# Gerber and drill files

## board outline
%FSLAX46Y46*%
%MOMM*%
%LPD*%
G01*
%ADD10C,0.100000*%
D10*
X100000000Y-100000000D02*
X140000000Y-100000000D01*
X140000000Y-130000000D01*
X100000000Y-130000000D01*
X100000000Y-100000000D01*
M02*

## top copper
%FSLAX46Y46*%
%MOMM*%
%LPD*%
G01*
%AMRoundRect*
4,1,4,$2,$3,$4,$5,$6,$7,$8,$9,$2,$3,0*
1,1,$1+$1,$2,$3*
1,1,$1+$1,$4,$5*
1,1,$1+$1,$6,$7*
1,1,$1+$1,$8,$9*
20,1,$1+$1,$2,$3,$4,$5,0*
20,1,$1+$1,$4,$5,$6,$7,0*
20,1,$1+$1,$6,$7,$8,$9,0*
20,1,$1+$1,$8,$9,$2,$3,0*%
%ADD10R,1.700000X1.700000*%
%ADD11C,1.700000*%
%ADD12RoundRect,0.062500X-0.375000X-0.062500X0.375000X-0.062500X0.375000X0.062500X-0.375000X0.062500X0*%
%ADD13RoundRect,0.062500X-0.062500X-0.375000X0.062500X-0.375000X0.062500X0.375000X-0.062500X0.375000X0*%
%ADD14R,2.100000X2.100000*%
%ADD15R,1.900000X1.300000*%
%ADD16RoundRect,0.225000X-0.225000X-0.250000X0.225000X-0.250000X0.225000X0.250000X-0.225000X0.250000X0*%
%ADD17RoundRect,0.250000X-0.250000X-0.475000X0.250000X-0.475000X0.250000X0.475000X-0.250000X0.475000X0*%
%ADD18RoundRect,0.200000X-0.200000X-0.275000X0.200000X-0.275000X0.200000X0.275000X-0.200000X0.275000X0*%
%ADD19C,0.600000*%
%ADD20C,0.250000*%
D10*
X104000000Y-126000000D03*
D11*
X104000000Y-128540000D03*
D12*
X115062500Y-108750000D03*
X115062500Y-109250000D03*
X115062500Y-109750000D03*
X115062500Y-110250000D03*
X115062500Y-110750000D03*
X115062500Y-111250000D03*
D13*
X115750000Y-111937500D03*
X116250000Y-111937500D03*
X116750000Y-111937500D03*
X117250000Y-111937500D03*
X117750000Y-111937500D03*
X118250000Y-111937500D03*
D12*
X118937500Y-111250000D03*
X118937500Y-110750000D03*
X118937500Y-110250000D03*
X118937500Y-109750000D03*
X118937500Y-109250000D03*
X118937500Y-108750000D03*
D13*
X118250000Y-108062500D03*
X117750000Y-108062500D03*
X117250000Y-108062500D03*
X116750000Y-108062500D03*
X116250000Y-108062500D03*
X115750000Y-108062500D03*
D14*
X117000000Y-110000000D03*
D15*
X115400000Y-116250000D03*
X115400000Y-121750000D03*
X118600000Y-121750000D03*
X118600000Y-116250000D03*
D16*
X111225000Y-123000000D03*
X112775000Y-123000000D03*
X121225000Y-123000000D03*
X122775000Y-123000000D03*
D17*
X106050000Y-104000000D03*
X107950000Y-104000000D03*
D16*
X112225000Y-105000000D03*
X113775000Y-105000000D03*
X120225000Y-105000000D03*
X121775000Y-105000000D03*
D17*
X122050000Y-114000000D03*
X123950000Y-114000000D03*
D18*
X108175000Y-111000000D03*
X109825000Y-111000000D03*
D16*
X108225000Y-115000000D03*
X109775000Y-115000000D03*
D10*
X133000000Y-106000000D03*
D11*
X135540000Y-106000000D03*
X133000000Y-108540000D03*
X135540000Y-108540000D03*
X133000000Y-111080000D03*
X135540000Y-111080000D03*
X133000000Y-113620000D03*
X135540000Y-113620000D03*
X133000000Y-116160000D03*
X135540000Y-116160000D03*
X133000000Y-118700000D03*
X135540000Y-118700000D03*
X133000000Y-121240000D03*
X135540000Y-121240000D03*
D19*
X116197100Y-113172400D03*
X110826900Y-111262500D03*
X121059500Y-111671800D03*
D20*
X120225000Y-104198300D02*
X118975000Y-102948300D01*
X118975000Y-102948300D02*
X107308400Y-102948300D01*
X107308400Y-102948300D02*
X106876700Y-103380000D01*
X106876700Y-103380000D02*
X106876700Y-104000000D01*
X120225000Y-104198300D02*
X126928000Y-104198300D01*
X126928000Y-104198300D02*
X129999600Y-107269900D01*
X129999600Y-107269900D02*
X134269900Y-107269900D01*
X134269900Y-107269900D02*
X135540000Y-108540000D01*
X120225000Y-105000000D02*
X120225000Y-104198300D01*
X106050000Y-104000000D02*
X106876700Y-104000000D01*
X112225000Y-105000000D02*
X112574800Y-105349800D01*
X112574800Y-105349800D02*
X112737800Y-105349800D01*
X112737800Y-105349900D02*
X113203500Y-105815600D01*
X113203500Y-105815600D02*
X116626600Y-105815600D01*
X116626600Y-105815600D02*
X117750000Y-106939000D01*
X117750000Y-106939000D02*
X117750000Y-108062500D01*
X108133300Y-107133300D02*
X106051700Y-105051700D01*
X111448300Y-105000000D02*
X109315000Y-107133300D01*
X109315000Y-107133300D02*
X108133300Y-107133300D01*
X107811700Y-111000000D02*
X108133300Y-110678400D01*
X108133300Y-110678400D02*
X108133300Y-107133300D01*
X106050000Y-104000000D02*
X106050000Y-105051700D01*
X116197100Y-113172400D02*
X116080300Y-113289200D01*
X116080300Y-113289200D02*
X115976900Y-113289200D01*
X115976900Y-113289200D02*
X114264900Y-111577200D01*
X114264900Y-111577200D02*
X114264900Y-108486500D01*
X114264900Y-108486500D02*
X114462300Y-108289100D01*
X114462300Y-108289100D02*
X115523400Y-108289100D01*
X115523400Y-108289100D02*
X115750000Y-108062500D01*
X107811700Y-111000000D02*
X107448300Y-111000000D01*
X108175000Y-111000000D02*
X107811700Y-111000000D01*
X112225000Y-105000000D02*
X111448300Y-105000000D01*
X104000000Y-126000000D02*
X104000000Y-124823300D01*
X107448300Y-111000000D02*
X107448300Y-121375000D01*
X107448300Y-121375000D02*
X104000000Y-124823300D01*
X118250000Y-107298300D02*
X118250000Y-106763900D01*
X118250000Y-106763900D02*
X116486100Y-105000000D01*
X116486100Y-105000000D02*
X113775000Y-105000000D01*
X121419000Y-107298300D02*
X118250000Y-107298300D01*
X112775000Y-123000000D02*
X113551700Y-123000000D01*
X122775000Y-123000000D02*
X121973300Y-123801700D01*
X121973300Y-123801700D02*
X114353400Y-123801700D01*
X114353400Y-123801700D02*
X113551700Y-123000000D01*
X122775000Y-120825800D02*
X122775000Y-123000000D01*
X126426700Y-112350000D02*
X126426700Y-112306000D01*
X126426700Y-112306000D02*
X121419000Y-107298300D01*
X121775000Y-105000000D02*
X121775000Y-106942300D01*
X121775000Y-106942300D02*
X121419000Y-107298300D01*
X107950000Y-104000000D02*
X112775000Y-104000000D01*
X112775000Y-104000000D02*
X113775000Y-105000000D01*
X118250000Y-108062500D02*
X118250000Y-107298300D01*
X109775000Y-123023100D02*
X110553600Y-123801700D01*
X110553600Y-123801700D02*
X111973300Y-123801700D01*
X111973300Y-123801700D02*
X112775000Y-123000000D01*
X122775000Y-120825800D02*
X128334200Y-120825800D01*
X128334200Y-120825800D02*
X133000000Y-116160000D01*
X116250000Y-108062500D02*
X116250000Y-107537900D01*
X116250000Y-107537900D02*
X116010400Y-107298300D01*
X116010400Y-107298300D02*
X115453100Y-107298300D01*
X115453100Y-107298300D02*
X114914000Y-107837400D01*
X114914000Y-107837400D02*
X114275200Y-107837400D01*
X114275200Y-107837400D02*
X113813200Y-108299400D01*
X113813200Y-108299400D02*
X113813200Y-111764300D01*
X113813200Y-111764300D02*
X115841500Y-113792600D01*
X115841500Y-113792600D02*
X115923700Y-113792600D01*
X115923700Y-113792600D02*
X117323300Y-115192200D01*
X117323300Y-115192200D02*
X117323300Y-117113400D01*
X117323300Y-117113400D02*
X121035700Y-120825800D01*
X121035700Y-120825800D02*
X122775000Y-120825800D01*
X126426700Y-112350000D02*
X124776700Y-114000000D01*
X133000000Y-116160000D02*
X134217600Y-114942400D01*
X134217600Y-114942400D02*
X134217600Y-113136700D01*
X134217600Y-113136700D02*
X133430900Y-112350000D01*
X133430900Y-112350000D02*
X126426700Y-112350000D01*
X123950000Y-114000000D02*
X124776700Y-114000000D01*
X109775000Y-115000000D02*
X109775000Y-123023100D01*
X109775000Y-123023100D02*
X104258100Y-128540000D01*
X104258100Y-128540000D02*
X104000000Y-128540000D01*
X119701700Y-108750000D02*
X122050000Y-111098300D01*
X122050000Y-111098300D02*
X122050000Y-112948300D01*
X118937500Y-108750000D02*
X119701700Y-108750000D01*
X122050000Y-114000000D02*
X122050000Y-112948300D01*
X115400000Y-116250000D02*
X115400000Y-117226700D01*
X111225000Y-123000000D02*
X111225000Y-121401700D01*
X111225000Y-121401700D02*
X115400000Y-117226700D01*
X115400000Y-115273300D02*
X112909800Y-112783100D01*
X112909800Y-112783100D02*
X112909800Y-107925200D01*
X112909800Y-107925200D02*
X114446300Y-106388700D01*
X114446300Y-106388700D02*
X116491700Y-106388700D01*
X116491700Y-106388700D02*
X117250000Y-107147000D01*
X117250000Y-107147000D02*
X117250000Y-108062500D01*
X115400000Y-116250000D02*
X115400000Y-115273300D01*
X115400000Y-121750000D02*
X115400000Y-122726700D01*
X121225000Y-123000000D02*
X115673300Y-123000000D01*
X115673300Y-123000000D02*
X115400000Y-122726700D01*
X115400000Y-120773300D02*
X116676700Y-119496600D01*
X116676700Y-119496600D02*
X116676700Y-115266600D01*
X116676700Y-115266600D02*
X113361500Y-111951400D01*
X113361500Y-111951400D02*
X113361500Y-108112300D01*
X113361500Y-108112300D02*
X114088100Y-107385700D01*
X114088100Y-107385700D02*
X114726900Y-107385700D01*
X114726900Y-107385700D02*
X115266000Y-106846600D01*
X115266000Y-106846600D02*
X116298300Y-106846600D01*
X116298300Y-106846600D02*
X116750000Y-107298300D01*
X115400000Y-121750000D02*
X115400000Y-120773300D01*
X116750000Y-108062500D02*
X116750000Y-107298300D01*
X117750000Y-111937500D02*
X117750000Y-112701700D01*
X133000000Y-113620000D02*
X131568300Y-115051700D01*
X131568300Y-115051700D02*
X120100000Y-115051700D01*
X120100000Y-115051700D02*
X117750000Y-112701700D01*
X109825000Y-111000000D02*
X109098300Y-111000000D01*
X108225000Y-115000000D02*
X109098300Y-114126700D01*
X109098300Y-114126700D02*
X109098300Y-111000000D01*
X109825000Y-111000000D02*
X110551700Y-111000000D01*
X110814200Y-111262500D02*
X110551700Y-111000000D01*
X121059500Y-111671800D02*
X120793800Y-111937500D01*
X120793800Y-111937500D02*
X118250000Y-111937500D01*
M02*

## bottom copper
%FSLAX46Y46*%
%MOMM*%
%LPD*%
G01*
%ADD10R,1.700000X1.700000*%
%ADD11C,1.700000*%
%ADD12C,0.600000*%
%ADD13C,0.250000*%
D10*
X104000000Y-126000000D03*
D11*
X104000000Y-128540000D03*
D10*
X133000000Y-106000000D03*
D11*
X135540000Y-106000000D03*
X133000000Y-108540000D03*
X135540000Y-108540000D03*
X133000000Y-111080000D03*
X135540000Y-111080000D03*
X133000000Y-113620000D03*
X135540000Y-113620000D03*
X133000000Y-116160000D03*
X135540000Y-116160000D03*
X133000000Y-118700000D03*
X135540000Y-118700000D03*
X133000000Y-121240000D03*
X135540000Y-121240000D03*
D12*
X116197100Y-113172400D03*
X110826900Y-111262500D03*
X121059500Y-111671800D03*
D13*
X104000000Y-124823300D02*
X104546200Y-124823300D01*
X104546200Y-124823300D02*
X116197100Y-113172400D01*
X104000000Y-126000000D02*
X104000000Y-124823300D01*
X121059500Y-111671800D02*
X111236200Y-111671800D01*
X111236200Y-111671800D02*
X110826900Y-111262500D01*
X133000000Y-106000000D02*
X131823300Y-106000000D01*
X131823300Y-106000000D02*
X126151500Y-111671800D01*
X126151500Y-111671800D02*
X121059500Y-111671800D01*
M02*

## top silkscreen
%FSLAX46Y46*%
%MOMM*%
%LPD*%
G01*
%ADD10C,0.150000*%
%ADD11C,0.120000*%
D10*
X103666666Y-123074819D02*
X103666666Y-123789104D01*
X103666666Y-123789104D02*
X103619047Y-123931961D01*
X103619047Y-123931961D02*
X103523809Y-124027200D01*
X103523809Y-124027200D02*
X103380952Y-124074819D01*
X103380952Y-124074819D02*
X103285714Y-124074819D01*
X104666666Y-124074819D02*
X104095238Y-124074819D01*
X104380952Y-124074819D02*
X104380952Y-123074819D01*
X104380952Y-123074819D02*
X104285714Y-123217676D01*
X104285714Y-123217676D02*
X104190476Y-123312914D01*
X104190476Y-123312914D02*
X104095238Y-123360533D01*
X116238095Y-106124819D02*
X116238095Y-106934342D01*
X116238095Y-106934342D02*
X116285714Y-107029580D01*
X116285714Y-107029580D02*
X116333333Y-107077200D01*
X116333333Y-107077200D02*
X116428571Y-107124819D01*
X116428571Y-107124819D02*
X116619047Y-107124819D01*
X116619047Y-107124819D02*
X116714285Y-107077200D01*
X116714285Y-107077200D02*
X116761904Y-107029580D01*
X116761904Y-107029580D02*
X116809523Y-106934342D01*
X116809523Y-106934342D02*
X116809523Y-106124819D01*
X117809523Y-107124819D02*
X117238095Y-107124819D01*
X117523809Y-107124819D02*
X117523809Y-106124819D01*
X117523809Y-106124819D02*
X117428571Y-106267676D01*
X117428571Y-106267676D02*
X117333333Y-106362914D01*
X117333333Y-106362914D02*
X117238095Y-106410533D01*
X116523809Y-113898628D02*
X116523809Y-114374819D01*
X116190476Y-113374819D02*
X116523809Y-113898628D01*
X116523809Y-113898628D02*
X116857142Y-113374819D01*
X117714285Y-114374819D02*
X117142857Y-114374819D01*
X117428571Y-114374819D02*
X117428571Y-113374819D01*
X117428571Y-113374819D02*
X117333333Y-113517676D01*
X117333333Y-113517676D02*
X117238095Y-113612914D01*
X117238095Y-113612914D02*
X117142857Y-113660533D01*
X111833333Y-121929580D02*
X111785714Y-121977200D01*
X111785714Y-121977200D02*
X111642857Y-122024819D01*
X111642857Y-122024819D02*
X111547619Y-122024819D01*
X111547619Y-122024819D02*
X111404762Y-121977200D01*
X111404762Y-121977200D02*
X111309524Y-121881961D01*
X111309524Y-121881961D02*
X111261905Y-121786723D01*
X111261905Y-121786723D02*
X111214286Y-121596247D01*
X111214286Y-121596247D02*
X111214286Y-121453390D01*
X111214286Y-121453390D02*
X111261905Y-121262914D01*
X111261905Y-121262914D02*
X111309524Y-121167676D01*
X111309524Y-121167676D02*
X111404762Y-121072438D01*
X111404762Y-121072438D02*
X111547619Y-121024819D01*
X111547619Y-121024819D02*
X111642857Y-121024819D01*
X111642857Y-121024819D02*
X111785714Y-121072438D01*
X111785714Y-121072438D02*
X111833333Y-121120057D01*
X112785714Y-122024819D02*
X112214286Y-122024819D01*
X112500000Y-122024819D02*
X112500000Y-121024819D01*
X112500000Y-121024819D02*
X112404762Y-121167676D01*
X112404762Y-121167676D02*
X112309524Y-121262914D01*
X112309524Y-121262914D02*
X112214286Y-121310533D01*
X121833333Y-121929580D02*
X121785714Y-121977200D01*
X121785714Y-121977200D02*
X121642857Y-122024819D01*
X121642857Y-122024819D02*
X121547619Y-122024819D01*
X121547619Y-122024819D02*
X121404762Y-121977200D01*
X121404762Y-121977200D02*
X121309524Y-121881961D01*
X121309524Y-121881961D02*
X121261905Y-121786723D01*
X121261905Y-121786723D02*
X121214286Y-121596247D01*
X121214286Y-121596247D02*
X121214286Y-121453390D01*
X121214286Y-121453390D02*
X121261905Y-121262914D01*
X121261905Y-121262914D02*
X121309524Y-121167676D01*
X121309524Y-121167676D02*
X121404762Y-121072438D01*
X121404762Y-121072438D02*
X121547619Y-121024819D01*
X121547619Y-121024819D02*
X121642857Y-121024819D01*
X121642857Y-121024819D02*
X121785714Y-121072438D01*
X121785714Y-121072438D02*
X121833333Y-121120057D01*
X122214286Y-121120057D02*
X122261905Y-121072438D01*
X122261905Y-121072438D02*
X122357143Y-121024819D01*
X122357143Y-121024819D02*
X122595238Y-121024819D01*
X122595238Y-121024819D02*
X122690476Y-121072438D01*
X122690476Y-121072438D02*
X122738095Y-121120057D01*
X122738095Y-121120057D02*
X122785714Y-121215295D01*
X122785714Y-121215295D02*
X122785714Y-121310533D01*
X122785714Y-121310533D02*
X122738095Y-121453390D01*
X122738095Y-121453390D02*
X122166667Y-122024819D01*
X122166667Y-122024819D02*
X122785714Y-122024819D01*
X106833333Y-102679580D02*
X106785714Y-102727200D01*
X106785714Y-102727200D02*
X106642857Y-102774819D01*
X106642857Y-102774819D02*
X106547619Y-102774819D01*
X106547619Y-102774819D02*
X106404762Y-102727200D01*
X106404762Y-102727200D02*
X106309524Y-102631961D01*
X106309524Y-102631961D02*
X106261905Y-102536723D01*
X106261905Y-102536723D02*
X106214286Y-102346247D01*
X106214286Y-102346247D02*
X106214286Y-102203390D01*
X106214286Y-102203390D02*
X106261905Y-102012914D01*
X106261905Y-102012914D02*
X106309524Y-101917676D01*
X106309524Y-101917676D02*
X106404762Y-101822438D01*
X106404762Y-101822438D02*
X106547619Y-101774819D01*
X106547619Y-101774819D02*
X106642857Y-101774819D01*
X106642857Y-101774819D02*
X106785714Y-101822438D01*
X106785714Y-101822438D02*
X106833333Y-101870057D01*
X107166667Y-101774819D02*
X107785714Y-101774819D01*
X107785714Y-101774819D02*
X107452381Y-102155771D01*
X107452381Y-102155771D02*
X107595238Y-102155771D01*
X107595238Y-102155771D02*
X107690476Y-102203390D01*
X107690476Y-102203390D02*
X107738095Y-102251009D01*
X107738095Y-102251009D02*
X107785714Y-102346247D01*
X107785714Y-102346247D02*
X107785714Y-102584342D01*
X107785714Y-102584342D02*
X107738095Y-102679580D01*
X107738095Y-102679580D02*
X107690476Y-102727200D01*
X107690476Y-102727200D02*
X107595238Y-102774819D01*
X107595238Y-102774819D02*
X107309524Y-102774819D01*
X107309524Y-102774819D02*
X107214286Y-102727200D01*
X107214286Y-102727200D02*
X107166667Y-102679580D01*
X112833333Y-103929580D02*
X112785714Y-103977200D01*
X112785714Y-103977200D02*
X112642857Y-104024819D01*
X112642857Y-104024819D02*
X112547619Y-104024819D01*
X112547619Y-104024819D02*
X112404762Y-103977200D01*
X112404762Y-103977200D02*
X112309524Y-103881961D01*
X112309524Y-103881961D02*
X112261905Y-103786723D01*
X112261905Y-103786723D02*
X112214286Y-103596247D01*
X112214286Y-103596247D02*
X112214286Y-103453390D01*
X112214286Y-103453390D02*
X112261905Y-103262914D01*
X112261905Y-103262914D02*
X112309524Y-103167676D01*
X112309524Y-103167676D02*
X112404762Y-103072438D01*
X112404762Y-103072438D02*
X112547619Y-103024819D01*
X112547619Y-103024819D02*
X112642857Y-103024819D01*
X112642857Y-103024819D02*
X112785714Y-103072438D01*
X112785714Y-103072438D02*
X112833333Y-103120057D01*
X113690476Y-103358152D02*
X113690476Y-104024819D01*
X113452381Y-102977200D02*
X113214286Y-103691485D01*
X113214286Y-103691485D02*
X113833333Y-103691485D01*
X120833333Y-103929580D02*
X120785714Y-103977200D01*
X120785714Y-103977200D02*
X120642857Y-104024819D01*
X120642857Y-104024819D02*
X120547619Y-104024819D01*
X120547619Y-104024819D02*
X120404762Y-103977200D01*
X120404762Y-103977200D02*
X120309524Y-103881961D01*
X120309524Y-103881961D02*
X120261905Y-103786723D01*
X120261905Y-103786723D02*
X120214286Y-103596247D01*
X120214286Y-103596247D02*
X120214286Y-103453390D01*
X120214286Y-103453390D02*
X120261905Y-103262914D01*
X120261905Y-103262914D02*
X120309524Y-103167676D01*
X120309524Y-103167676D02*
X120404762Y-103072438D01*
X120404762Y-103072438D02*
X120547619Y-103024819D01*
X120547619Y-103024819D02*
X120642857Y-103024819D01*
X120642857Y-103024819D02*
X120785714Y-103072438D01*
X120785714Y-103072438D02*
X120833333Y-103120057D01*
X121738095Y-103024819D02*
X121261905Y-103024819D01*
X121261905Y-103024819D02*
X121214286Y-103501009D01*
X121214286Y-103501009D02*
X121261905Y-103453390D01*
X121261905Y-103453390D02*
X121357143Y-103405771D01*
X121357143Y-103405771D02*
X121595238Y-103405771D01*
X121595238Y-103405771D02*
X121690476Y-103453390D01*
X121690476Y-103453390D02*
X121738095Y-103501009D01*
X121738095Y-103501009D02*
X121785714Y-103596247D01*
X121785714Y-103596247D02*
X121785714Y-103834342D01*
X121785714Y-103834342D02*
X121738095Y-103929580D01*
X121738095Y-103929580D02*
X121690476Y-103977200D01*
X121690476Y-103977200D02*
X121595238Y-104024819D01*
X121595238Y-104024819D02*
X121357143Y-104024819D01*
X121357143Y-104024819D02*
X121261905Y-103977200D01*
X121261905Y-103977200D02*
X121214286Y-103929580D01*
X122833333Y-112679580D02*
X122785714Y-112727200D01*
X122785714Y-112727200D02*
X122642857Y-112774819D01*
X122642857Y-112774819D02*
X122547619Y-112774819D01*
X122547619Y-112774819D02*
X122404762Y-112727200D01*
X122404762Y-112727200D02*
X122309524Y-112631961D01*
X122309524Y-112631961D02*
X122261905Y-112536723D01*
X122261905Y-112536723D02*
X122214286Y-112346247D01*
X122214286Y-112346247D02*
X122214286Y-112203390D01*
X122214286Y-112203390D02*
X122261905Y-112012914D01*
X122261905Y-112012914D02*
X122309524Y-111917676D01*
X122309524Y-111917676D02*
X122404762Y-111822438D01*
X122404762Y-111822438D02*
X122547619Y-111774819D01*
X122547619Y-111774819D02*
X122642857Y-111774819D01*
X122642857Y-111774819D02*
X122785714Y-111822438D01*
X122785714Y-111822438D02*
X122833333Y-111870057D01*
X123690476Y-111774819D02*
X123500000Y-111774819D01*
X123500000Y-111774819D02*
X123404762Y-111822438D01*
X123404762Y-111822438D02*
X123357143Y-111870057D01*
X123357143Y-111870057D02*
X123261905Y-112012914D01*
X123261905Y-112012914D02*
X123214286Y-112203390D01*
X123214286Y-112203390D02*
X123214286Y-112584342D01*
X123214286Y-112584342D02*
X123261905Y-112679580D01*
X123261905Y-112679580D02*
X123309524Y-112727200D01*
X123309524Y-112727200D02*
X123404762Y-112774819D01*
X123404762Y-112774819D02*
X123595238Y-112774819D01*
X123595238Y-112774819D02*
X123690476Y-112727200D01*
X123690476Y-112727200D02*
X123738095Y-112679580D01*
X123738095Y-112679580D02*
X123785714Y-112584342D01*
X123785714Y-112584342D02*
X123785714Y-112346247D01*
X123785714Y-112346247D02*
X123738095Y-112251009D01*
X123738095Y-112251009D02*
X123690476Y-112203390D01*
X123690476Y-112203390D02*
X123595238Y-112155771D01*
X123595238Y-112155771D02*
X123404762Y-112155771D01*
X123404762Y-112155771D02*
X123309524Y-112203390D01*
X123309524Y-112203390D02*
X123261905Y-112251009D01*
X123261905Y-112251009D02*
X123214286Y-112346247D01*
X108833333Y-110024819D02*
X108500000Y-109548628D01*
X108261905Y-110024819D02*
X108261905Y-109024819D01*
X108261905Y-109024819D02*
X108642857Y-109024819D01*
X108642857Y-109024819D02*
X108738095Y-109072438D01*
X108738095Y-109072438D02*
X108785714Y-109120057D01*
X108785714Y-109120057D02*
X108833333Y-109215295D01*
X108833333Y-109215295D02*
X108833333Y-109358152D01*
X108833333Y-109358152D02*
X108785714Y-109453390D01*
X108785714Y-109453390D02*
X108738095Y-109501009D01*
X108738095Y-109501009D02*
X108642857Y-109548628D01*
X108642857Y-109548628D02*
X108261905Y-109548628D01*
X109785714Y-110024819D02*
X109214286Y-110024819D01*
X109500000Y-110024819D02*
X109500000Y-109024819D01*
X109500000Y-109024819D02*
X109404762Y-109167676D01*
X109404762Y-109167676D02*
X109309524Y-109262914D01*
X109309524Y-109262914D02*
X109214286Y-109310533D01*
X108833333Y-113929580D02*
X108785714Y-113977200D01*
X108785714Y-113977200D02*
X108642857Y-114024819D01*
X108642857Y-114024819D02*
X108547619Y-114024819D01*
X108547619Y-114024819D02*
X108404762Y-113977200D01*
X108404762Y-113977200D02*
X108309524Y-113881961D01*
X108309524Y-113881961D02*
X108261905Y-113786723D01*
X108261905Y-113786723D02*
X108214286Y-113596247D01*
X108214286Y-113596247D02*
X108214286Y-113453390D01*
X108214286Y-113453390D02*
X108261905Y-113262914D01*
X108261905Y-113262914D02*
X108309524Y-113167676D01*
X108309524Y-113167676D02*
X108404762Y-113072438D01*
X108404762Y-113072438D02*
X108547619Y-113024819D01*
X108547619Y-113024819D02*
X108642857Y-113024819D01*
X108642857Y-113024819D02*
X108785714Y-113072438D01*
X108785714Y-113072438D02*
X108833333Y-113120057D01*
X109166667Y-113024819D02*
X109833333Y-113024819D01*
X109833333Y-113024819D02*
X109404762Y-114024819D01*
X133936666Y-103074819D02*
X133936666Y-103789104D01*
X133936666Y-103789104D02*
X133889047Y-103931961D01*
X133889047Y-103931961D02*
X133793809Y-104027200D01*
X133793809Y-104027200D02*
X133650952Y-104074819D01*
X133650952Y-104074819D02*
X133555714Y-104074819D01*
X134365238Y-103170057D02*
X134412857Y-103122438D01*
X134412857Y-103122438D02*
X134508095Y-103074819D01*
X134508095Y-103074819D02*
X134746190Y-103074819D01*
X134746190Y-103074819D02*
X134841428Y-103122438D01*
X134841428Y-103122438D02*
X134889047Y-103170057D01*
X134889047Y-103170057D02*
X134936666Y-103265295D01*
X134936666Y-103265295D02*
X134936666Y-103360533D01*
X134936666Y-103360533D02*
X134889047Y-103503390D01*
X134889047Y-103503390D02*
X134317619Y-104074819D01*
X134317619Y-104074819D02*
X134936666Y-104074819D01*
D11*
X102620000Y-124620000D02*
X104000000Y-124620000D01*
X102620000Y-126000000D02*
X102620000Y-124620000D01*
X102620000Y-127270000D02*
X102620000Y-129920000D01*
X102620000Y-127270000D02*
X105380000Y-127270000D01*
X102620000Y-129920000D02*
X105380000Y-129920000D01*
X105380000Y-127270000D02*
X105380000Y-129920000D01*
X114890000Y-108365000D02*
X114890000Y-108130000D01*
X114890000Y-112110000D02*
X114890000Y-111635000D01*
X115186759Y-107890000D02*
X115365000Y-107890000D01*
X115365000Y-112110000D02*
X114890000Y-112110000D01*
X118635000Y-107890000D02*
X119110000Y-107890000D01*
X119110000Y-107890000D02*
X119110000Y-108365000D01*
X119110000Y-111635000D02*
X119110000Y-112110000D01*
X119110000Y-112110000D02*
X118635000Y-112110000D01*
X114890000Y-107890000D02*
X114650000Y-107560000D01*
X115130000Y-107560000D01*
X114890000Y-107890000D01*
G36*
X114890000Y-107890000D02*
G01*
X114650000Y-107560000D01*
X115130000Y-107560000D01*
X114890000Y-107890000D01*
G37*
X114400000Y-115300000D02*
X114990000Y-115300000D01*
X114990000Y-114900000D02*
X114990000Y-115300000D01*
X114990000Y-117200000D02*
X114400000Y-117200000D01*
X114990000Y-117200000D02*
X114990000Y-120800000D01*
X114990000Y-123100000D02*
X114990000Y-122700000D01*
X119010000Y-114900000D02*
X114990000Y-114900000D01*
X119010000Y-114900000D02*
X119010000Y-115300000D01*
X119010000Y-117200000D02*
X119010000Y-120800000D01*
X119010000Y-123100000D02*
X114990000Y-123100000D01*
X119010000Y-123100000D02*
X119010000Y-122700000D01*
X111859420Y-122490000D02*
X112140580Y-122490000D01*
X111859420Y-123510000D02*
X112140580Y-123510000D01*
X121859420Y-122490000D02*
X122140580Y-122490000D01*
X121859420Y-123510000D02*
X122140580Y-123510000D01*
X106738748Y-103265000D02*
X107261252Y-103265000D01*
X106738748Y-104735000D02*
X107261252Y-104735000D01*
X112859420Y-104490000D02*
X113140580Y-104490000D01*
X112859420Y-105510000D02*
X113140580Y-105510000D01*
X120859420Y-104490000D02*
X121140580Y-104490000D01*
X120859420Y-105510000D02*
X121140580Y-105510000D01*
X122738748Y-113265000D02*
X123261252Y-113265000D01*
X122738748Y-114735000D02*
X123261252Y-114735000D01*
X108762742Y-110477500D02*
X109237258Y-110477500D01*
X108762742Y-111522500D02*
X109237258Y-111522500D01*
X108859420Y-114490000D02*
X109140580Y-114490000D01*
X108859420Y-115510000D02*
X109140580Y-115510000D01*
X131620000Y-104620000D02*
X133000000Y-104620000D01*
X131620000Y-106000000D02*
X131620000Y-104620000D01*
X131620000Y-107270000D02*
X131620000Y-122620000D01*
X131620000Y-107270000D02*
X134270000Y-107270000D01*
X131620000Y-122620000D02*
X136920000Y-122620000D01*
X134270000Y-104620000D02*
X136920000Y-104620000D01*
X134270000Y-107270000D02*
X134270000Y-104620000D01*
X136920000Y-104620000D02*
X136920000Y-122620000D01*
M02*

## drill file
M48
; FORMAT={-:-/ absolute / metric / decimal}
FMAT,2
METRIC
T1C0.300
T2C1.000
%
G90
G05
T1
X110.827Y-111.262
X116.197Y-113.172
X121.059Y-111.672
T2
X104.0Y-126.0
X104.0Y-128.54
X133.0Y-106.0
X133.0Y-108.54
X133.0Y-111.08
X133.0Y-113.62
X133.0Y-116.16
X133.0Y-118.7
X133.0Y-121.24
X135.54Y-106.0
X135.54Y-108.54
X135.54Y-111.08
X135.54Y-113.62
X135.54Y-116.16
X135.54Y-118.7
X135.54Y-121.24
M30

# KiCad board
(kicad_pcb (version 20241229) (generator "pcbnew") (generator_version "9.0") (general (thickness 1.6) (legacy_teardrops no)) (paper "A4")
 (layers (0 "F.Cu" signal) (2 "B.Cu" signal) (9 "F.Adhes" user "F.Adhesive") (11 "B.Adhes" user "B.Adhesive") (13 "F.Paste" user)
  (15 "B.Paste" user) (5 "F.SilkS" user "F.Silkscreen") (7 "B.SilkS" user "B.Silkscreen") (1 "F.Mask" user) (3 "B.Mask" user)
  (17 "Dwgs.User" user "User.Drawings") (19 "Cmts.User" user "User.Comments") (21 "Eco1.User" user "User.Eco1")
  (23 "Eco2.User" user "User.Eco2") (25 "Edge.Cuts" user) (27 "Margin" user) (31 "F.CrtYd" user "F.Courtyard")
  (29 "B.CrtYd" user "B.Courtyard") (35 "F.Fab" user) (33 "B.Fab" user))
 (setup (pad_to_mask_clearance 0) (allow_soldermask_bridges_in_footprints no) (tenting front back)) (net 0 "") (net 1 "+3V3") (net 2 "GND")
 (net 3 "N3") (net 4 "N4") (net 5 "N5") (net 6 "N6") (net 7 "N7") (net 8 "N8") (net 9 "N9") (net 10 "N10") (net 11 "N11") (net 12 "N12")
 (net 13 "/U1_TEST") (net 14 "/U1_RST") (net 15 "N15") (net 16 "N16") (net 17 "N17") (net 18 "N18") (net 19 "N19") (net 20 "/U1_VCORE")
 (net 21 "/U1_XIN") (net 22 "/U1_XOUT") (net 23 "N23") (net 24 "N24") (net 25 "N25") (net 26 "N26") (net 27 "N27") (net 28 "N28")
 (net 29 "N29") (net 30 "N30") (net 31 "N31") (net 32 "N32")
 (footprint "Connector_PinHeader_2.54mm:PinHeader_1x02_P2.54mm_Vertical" (layer "F.Cu") (at 104 126)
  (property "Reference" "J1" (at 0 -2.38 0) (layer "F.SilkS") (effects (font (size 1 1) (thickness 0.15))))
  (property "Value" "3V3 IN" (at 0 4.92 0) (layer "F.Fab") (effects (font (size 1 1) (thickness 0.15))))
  (fp_line (start -1.38 -1.38) (end 0 -1.38) (stroke (width 0.12) (type solid)) (layer "F.SilkS"))
  (fp_line (start -1.38 0) (end -1.38 -1.38) (stroke (width 0.12) (type solid)) (layer "F.SilkS"))
  (fp_line (start -1.38 1.27) (end -1.38 3.92) (stroke (width 0.12) (type solid)) (layer "F.SilkS"))
  (fp_line (start -1.38 1.27) (end 1.38 1.27) (stroke (width 0.12) (type solid)) (layer "F.SilkS"))
  (fp_line (start -1.38 3.92) (end 1.38 3.92) (stroke (width 0.12) (type solid)) (layer "F.SilkS"))
  (fp_line (start 1.38 1.27) (end 1.38 3.92) (stroke (width 0.12) (type solid)) (layer "F.SilkS"))
  (pad "1" thru_hole rect (at 0 0) (size 1.7 1.7) (drill 1) (layers "*.Cu" "*.Mask") (remove_unused_layers no) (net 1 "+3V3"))
  (pad "2" thru_hole circle (at 0 2.54) (size 1.7 1.7) (drill 1) (layers "*.Cu" "*.Mask") (remove_unused_layers no) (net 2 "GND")))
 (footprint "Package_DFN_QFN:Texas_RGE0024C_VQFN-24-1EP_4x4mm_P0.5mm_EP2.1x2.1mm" (layer "F.Cu") (at 117 110)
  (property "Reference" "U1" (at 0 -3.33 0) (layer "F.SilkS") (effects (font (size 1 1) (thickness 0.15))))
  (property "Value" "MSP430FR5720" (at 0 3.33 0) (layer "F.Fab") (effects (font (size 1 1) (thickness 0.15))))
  (fp_line (start -2.11 -1.635) (end -2.11 -1.87) (stroke (width 0.12) (type solid)) (layer "F.SilkS"))
  (fp_line (start -2.11 2.11) (end -2.11 1.635) (stroke (width 0.12) (type solid)) (layer "F.SilkS"))
  (fp_line (start -1.813241 -2.11) (end -1.635 -2.11) (stroke (width 0.12) (type solid)) (layer "F.SilkS"))
  (fp_line (start -1.635 2.11) (end -2.11 2.11) (stroke (width 0.12) (type solid)) (layer "F.SilkS"))
  (fp_line (start 1.635 -2.11) (end 2.11 -2.11) (stroke (width 0.12) (type solid)) (layer "F.SilkS"))
  (fp_line (start 2.11 -2.11) (end 2.11 -1.635) (stroke (width 0.12) (type solid)) (layer "F.SilkS"))
  (fp_line (start 2.11 1.635) (end 2.11 2.11) (stroke (width 0.12) (type solid)) (layer "F.SilkS"))
  (fp_line (start 2.11 2.11) (end 1.635 2.11) (stroke (width 0.12) (type solid)) (layer "F.SilkS"))
  (fp_poly (pts (xy -2.11 -2.11) (xy -2.35 -2.44) (xy -1.87 -2.44)) (stroke (width 0.12) (type solid)) (fill yes) (layer "F.SilkS"))
  (pad "" smd roundrect (at -0.525 -0.525) (size 0.85 0.85) (layers "F.Paste") (roundrect_rratio 0.25))
  (pad "" smd roundrect (at -0.525 0.525) (size 0.85 0.85) (layers "F.Paste") (roundrect_rratio 0.25))
  (pad "" smd roundrect (at 0.525 -0.525) (size 0.85 0.85) (layers "F.Paste") (roundrect_rratio 0.25))
  (pad "" smd roundrect (at 0.525 0.525) (size 0.85 0.85) (layers "F.Paste") (roundrect_rratio 0.25))
  (pad "1" smd roundrect (at -1.9375 -1.25) (size 0.875 0.25) (layers "F.Cu" "F.Mask" "F.Paste") (roundrect_rratio 0.25) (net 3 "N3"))
  (pad "2" smd roundrect (at -1.9375 -0.75) (size 0.875 0.25) (layers "F.Cu" "F.Mask" "F.Paste") (roundrect_rratio 0.25) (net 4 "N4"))
  (pad "3" smd roundrect (at -1.9375 -0.25) (size 0.875 0.25) (layers "F.Cu" "F.Mask" "F.Paste") (roundrect_rratio 0.25) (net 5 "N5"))
  (pad "4" smd roundrect (at -1.9375 0.25) (size 0.875 0.25) (layers "F.Cu" "F.Mask" "F.Paste") (roundrect_rratio 0.25) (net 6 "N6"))
  (pad "5" smd roundrect (at -1.9375 0.75) (size 0.875 0.25) (layers "F.Cu" "F.Mask" "F.Paste") (roundrect_rratio 0.25) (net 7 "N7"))
  (pad "6" smd roundrect (at -1.9375 1.25) (size 0.875 0.25) (layers "F.Cu" "F.Mask" "F.Paste") (roundrect_rratio 0.25) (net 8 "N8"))
  (pad "7" smd roundrect (at -1.25 1.9375) (size 0.25 0.875) (layers "F.Cu" "F.Mask" "F.Paste") (roundrect_rratio 0.25) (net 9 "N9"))
  (pad "8" smd roundrect (at -0.75 1.9375) (size 0.25 0.875) (layers "F.Cu" "F.Mask" "F.Paste") (roundrect_rratio 0.25) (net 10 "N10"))
  (pad "9" smd roundrect (at -0.25 1.9375) (size 0.25 0.875) (layers "F.Cu" "F.Mask" "F.Paste") (roundrect_rratio 0.25) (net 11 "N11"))
  (pad "10" smd roundrect (at 0.25 1.9375) (size 0.25 0.875) (layers "F.Cu" "F.Mask" "F.Paste") (roundrect_rratio 0.25) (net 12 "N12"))
  (pad "11" smd roundrect (at 0.75 1.9375) (size 0.25 0.875) (layers "F.Cu" "F.Mask" "F.Paste") (roundrect_rratio 0.25) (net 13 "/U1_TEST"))
  (pad "12" smd roundrect (at 1.25 1.9375) (size 0.25 0.875) (layers "F.Cu" "F.Mask" "F.Paste") (roundrect_rratio 0.25) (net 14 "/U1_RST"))
  (pad "13" smd roundrect (at 1.9375 1.25) (size 0.875 0.25) (layers "F.Cu" "F.Mask" "F.Paste") (roundrect_rratio 0.25) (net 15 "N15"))
  (pad "14" smd roundrect (at 1.9375 0.75) (size 0.875 0.25) (layers "F.Cu" "F.Mask" "F.Paste") (roundrect_rratio 0.25) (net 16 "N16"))
  (pad "15" smd roundrect (at 1.9375 0.25) (size 0.875 0.25) (layers "F.Cu" "F.Mask" "F.Paste") (roundrect_rratio 0.25) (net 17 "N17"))
  (pad "16" smd roundrect (at 1.9375 -0.25) (size 0.875 0.25) (layers "F.Cu" "F.Mask" "F.Paste") (roundrect_rratio 0.25) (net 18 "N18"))
  (pad "17" smd roundrect (at 1.9375 -0.75) (size 0.875 0.25) (layers "F.Cu" "F.Mask" "F.Paste") (roundrect_rratio 0.25) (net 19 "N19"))
  (pad "18" smd roundrect (at 1.9375 -1.25) (size 0.875 0.25) (layers "F.Cu" "F.Mask" "F.Paste") (roundrect_rratio 0.25)
   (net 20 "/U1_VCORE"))
  (pad "19" smd roundrect (at 1.25 -1.9375) (size 0.25 0.875) (layers "F.Cu" "F.Mask" "F.Paste") (roundrect_rratio 0.25) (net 2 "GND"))
  (pad "20" smd roundrect (at 0.75 -1.9375) (size 0.25 0.875) (layers "F.Cu" "F.Mask" "F.Paste") (roundrect_rratio 0.25) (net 1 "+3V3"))
  (pad "21" smd roundrect (at 0.25 -1.9375) (size 0.25 0.875) (layers "F.Cu" "F.Mask" "F.Paste") (roundrect_rratio 0.25) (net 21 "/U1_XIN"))
  (pad "22" smd roundrect (at -0.25 -1.9375) (size 0.25 0.875) (layers "F.Cu" "F.Mask" "F.Paste") (roundrect_rratio 0.25)
   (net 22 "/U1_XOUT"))
  (pad "23" smd roundrect (at -0.75 -1.9375) (size 0.25 0.875) (layers "F.Cu" "F.Mask" "F.Paste") (roundrect_rratio 0.25) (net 2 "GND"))
  (pad "24" smd roundrect (at -1.25 -1.9375) (size 0.25 0.875) (layers "F.Cu" "F.Mask" "F.Paste") (roundrect_rratio 0.25) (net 1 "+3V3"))
  (pad "25" smd rect (at 0 0) (size 2.1 2.1) (layers "F.Cu" "F.Mask") (zone_connect 2)))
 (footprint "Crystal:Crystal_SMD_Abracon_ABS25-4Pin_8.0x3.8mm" (layer "F.Cu") (at 117 119)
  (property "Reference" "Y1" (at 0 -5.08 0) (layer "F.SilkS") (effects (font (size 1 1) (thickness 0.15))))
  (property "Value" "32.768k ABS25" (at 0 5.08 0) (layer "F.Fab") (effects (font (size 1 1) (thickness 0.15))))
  (fp_line (start -2.6 -3.7) (end -2.01 -3.7) (stroke (width 0.12) (type solid)) (layer "F.SilkS"))
  (fp_line (start -2.01 -4.1) (end -2.01 -3.7) (stroke (width 0.12) (type solid)) (layer "F.SilkS"))
  (fp_line (start -2.01 -1.8) (end -2.6 -1.8) (stroke (width 0.12) (type solid)) (layer "F.SilkS"))
  (fp_line (start -2.01 -1.8) (end -2.01 1.8) (stroke (width 0.12) (type solid)) (layer "F.SilkS"))
  (fp_line (start -2.01 4.1) (end -2.01 3.7) (stroke (width 0.12) (type solid)) (layer "F.SilkS"))
  (fp_line (start 2.01 -4.1) (end -2.01 -4.1) (stroke (width 0.12) (type solid)) (layer "F.SilkS"))
  (fp_line (start 2.01 -4.1) (end 2.01 -3.7) (stroke (width 0.12) (type solid)) (layer "F.SilkS"))
  (fp_line (start 2.01 -1.8) (end 2.01 1.8) (stroke (width 0.12) (type solid)) (layer "F.SilkS"))
  (fp_line (start 2.01 4.1) (end -2.01 4.1) (stroke (width 0.12) (type solid)) (layer "F.SilkS"))
  (fp_line (start 2.01 4.1) (end 2.01 3.7) (stroke (width 0.12) (type solid)) (layer "F.SilkS"))
  (pad "1" smd rect (at -1.6 -2.75 270) (size 1.3 1.9) (layers "F.Cu" "F.Mask" "F.Paste") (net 21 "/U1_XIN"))
  (pad "2" smd rect (at -1.6 2.75 270) (size 1.3 1.9) (layers "F.Cu" "F.Mask" "F.Paste") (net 22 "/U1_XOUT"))
  (pad "3" smd rect (at 1.6 2.75 270) (size 1.3 1.9) (layers "F.Cu" "F.Mask" "F.Paste"))
  (pad "4" smd rect (at 1.6 -2.75 270) (size 1.3 1.9) (layers "F.Cu" "F.Mask" "F.Paste")))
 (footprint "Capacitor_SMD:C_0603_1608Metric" (layer "F.Cu") (at 112 123)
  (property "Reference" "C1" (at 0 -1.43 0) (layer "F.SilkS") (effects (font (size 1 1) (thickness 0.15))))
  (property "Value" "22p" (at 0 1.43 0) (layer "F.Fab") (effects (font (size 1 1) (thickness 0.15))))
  (fp_line (start -0.14058 -0.51) (end 0.14058 -0.51) (stroke (width 0.12) (type solid)) (layer "F.SilkS"))
  (fp_line (start -0.14058 0.51) (end 0.14058 0.51) (stroke (width 0.12) (type solid)) (layer "F.SilkS"))
  (pad "1" smd roundrect (at -0.775 0) (size 0.9 0.95) (layers "F.Cu" "F.Mask" "F.Paste") (roundrect_rratio 0.25) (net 21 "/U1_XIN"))
  (pad "2" smd roundrect (at 0.775 0) (size 0.9 0.95) (layers "F.Cu" "F.Mask" "F.Paste") (roundrect_rratio 0.25) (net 2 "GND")))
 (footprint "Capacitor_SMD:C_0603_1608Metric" (layer "F.Cu") (at 122 123)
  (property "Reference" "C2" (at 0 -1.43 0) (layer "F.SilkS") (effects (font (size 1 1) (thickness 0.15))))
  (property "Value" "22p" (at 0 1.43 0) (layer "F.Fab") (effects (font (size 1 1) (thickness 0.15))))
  (fp_line (start -0.14058 -0.51) (end 0.14058 -0.51) (stroke (width 0.12) (type solid)) (layer "F.SilkS"))
  (fp_line (start -0.14058 0.51) (end 0.14058 0.51) (stroke (width 0.12) (type solid)) (layer "F.SilkS"))
  (pad "1" smd roundrect (at -0.775 0) (size 0.9 0.95) (layers "F.Cu" "F.Mask" "F.Paste") (roundrect_rratio 0.25) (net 22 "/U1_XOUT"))
  (pad "2" smd roundrect (at 0.775 0) (size 0.9 0.95) (layers "F.Cu" "F.Mask" "F.Paste") (roundrect_rratio 0.25) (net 2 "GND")))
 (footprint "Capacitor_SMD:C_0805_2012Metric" (layer "F.Cu") (at 107 104)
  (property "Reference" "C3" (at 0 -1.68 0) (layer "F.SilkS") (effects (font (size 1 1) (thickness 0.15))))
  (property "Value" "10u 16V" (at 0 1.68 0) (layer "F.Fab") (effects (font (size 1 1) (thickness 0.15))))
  (fp_line (start -0.261252 -0.735) (end 0.261252 -0.735) (stroke (width 0.12) (type solid)) (layer "F.SilkS"))
  (fp_line (start -0.261252 0.735) (end 0.261252 0.735) (stroke (width 0.12) (type solid)) (layer "F.SilkS"))
  (pad "1" smd roundrect (at -0.95 0) (size 1 1.45) (layers "F.Cu" "F.Mask" "F.Paste") (roundrect_rratio 0.25) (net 1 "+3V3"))
  (pad "2" smd roundrect (at 0.95 0) (size 1 1.45) (layers "F.Cu" "F.Mask" "F.Paste") (roundrect_rratio 0.25) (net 2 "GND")))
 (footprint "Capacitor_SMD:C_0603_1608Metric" (layer "F.Cu") (at 113 105)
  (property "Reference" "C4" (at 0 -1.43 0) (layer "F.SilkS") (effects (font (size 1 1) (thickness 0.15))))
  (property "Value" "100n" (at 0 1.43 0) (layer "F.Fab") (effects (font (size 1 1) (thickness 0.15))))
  (fp_line (start -0.14058 -0.51) (end 0.14058 -0.51) (stroke (width 0.12) (type solid)) (layer "F.SilkS"))
  (fp_line (start -0.14058 0.51) (end 0.14058 0.51) (stroke (width 0.12) (type solid)) (layer "F.SilkS"))
  (pad "1" smd roundrect (at -0.775 0) (size 0.9 0.95) (layers "F.Cu" "F.Mask" "F.Paste") (roundrect_rratio 0.25) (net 1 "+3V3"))
  (pad "2" smd roundrect (at 0.775 0) (size 0.9 0.95) (layers "F.Cu" "F.Mask" "F.Paste") (roundrect_rratio 0.25) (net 2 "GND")))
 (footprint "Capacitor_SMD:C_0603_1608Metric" (layer "F.Cu") (at 121 105)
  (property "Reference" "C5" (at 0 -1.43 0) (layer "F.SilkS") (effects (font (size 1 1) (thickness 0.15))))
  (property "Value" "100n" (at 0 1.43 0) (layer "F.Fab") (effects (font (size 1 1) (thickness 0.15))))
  (fp_line (start -0.14058 -0.51) (end 0.14058 -0.51) (stroke (width 0.12) (type solid)) (layer "F.SilkS"))
  (fp_line (start -0.14058 0.51) (end 0.14058 0.51) (stroke (width 0.12) (type solid)) (layer "F.SilkS"))
  (pad "1" smd roundrect (at -0.775 0) (size 0.9 0.95) (layers "F.Cu" "F.Mask" "F.Paste") (roundrect_rratio 0.25) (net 1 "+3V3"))
  (pad "2" smd roundrect (at 0.775 0) (size 0.9 0.95) (layers "F.Cu" "F.Mask" "F.Paste") (roundrect_rratio 0.25) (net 2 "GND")))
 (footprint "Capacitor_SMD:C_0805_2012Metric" (layer "F.Cu") (at 123 114)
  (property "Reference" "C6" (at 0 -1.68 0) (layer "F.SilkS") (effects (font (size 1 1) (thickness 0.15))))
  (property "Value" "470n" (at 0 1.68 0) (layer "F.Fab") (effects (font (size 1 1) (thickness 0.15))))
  (fp_line (start -0.261252 -0.735) (end 0.261252 -0.735) (stroke (width 0.12) (type solid)) (layer "F.SilkS"))
  (fp_line (start -0.261252 0.735) (end 0.261252 0.735) (stroke (width 0.12) (type solid)) (layer "F.SilkS"))
  (pad "1" smd roundrect (at -0.95 0) (size 1 1.45) (layers "F.Cu" "F.Mask" "F.Paste") (roundrect_rratio 0.25) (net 20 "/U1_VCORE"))
  (pad "2" smd roundrect (at 0.95 0) (size 1 1.45) (layers "F.Cu" "F.Mask" "F.Paste") (roundrect_rratio 0.25) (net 2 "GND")))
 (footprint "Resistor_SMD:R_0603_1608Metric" (layer "F.Cu") (at 109 111)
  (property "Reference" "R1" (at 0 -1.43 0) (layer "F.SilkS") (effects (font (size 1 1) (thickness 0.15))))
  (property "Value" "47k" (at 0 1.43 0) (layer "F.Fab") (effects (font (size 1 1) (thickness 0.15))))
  (fp_line (start -0.237258 -0.5225) (end 0.237258 -0.5225) (stroke (width 0.12) (type solid)) (layer "F.SilkS"))
  (fp_line (start -0.237258 0.5225) (end 0.237258 0.5225) (stroke (width 0.12) (type solid)) (layer "F.SilkS"))
  (pad "1" smd roundrect (at -0.825 0) (size 0.8 0.95) (layers "F.Cu" "F.Mask" "F.Paste") (roundrect_rratio 0.25) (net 1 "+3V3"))
  (pad "2" smd roundrect (at 0.825 0) (size 0.8 0.95) (layers "F.Cu" "F.Mask" "F.Paste") (roundrect_rratio 0.25) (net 14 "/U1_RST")))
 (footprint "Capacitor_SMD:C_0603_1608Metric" (layer "F.Cu") (at 109 115)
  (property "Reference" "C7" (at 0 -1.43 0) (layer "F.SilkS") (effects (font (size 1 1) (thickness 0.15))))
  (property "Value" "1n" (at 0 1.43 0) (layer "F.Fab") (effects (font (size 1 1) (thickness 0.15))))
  (fp_line (start -0.14058 -0.51) (end 0.14058 -0.51) (stroke (width 0.12) (type solid)) (layer "F.SilkS"))
  (fp_line (start -0.14058 0.51) (end 0.14058 0.51) (stroke (width 0.12) (type solid)) (layer "F.SilkS"))
  (pad "1" smd roundrect (at -0.775 0) (size 0.9 0.95) (layers "F.Cu" "F.Mask" "F.Paste") (roundrect_rratio 0.25) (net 14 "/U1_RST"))
  (pad "2" smd roundrect (at 0.775 0) (size 0.9 0.95) (layers "F.Cu" "F.Mask" "F.Paste") (roundrect_rratio 0.25) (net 2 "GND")))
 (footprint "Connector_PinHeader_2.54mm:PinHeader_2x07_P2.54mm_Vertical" (layer "F.Cu") (at 133 106)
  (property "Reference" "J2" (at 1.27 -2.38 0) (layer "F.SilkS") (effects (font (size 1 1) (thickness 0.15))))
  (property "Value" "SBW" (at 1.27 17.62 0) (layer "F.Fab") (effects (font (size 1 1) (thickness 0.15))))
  (fp_line (start -1.38 -1.38) (end 0 -1.38) (stroke (width 0.12) (type solid)) (layer "F.SilkS"))
  (fp_line (start -1.38 0) (end -1.38 -1.38) (stroke (width 0.12) (type solid)) (layer "F.SilkS"))
  (fp_line (start -1.38 1.27) (end -1.38 16.62) (stroke (width 0.12) (type solid)) (layer "F.SilkS"))
  (fp_line (start -1.38 1.27) (end 1.27 1.27) (stroke (width 0.12) (type solid)) (layer "F.SilkS"))
  (fp_line (start -1.38 16.62) (end 3.92 16.62) (stroke (width 0.12) (type solid)) (layer "F.SilkS"))
  (fp_line (start 1.27 -1.38) (end 3.92 -1.38) (stroke (width 0.12) (type solid)) (layer "F.SilkS"))
  (fp_line (start 1.27 1.27) (end 1.27 -1.38) (stroke (width 0.12) (type solid)) (layer "F.SilkS"))
  (fp_line (start 3.92 -1.38) (end 3.92 16.62) (stroke (width 0.12) (type solid)) (layer "F.SilkS"))
  (pad "1" thru_hole rect (at 0 0) (size 1.7 1.7) (drill 1) (layers "*.Cu" "*.Mask") (remove_unused_layers no) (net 14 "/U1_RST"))
  (pad "2" thru_hole circle (at 2.54 0) (size 1.7 1.7) (drill 1) (layers "*.Cu" "*.Mask") (remove_unused_layers no) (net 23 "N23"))
  (pad "3" thru_hole circle (at 0 2.54) (size 1.7 1.7) (drill 1) (layers "*.Cu" "*.Mask") (remove_unused_layers no) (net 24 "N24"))
  (pad "4" thru_hole circle (at 2.54 2.54) (size 1.7 1.7) (drill 1) (layers "*.Cu" "*.Mask") (remove_unused_layers no) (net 1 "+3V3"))
  (pad "5" thru_hole circle (at 0 5.08) (size 1.7 1.7) (drill 1) (layers "*.Cu" "*.Mask") (remove_unused_layers no) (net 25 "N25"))
  (pad "6" thru_hole circle (at 2.54 5.08) (size 1.7 1.7) (drill 1) (layers "*.Cu" "*.Mask") (remove_unused_layers no) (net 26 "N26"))
  (pad "7" thru_hole circle (at 0 7.62) (size 1.7 1.7) (drill 1) (layers "*.Cu" "*.Mask") (remove_unused_layers no) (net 13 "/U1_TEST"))
  (pad "8" thru_hole circle (at 2.54 7.62) (size 1.7 1.7) (drill 1) (layers "*.Cu" "*.Mask") (remove_unused_layers no) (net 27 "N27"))
  (pad "9" thru_hole circle (at 0 10.16) (size 1.7 1.7) (drill 1) (layers "*.Cu" "*.Mask") (remove_unused_layers no) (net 2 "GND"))
  (pad "10" thru_hole circle (at 2.54 10.16) (size 1.7 1.7) (drill 1) (layers "*.Cu" "*.Mask") (remove_unused_layers no) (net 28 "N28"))
  (pad "11" thru_hole circle (at 0 12.7) (size 1.7 1.7) (drill 1) (layers "*.Cu" "*.Mask") (remove_unused_layers no) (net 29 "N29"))
  (pad "12" thru_hole circle (at 2.54 12.7) (size 1.7 1.7) (drill 1) (layers "*.Cu" "*.Mask") (remove_unused_layers no) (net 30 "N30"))
  (pad "13" thru_hole circle (at 0 15.24) (size 1.7 1.7) (drill 1) (layers "*.Cu" "*.Mask") (remove_unused_layers no) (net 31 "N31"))
  (pad "14" thru_hole circle (at 2.54 15.24) (size 1.7 1.7) (drill 1) (layers "*.Cu" "*.Mask") (remove_unused_layers no) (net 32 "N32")))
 (gr_rect (start 100 100) (end 140 130) (stroke (width 0.1) (type default)) (fill no) (layer "Edge.Cuts"))
 (segment (start 120.225 104.1983) (end 118.975 102.9483) (width 0.25) (layer "F.Cu") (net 1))
 (segment (start 118.975 102.9483) (end 107.3084 102.9483) (width 0.25) (layer "F.Cu") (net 1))
 (segment (start 107.3084 102.9483) (end 106.8767 103.38) (width 0.25) (layer "F.Cu") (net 1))
 (segment (start 106.8767 103.38) (end 106.8767 104) (width 0.25) (layer "F.Cu") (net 1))
 (segment (start 120.225 104.1983) (end 126.928 104.1983) (width 0.25) (layer "F.Cu") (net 1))
 (segment (start 126.928 104.1983) (end 129.9996 107.2699) (width 0.25) (layer "F.Cu") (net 1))
 (segment (start 129.9996 107.2699) (end 134.2699 107.2699) (width 0.25) (layer "F.Cu") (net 1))
 (segment (start 134.2699 107.2699) (end 135.54 108.54) (width 0.25) (layer "F.Cu") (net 1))
 (segment (start 120.225 105) (end 120.225 104.1983) (width 0.25) (layer "F.Cu") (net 1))
 (segment (start 106.05 104) (end 106.8767 104) (width 0.25) (layer "F.Cu") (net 1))
 (segment (start 112.225 105) (end 112.5748 105.3498) (width 0.25) (layer "F.Cu") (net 1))
 (segment (start 112.5748 105.3498) (end 112.7378 105.3498) (width 0.25) (layer "F.Cu") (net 1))
 (segment (start 112.7378 105.3499) (end 113.2035 105.8156) (width 0.25) (layer "F.Cu") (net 1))
 (segment (start 113.2035 105.8156) (end 116.6266 105.8156) (width 0.25) (layer "F.Cu") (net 1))
 (segment (start 116.6266 105.8156) (end 117.75 106.939) (width 0.25) (layer "F.Cu") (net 1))
 (segment (start 117.75 106.939) (end 117.75 108.0625) (width 0.25) (layer "F.Cu") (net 1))
 (segment (start 108.1333 107.1333) (end 106.0517 105.0517) (width 0.25) (layer "F.Cu") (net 1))
 (segment (start 111.4483 105) (end 109.315 107.1333) (width 0.25) (layer "F.Cu") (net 1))
 (segment (start 109.315 107.1333) (end 108.1333 107.1333) (width 0.25) (layer "F.Cu") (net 1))
 (segment (start 107.8117 111) (end 108.1333 110.6784) (width 0.25) (layer "F.Cu") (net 1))
 (segment (start 108.1333 110.6784) (end 108.1333 107.1333) (width 0.25) (layer "F.Cu") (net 1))
 (segment (start 106.05 104) (end 106.05 105.0517) (width 0.25) (layer "F.Cu") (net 1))
 (segment (start 116.1971 113.1724) (end 116.0803 113.2892) (width 0.25) (layer "F.Cu") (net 1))
 (segment (start 116.0803 113.2892) (end 115.9769 113.2892) (width 0.25) (layer "F.Cu") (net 1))
 (segment (start 115.9769 113.2892) (end 114.2649 111.5772) (width 0.25) (layer "F.Cu") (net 1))
 (segment (start 114.2649 111.5772) (end 114.2649 108.4865) (width 0.25) (layer "F.Cu") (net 1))
 (segment (start 114.2649 108.4865) (end 114.4623 108.2891) (width 0.25) (layer "F.Cu") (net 1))
 (segment (start 114.4623 108.2891) (end 115.5234 108.2891) (width 0.25) (layer "F.Cu") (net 1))
 (segment (start 115.5234 108.2891) (end 115.75 108.0625) (width 0.25) (layer "F.Cu") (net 1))
 (segment (start 104 124.8233) (end 104.5462 124.8233) (width 0.25) (layer "B.Cu") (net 1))
 (segment (start 104.5462 124.8233) (end 116.1971 113.1724) (width 0.25) (layer "B.Cu") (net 1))
 (segment (start 104 126) (end 104 124.8233) (width 0.25) (layer "B.Cu") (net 1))
 (segment (start 107.8117 111) (end 107.4483 111) (width 0.25) (layer "F.Cu") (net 1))
 (segment (start 108.175 111) (end 107.8117 111) (width 0.25) (layer "F.Cu") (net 1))
 (segment (start 112.225 105) (end 111.4483 105) (width 0.25) (layer "F.Cu") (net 1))
 (segment (start 104 126) (end 104 124.8233) (width 0.25) (layer "F.Cu") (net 1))
 (segment (start 107.4483 111) (end 107.4483 121.375) (width 0.25) (layer "F.Cu") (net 1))
 (segment (start 107.4483 121.375) (end 104 124.8233) (width 0.25) (layer "F.Cu") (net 1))
 (segment (start 118.25 107.2983) (end 118.25 106.7639) (width 0.25) (layer "F.Cu") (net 2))
 (segment (start 118.25 106.7639) (end 116.4861 105) (width 0.25) (layer "F.Cu") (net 2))
 (segment (start 116.4861 105) (end 113.775 105) (width 0.25) (layer "F.Cu") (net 2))
 (segment (start 121.419 107.2983) (end 118.25 107.2983) (width 0.25) (layer "F.Cu") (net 2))
 (segment (start 112.775 123) (end 113.5517 123) (width 0.25) (layer "F.Cu") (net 2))
 (segment (start 122.775 123) (end 121.9733 123.8017) (width 0.25) (layer "F.Cu") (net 2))
 (segment (start 121.9733 123.8017) (end 114.3534 123.8017) (width 0.25) (layer "F.Cu") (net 2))
 (segment (start 114.3534 123.8017) (end 113.5517 123) (width 0.25) (layer "F.Cu") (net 2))
 (segment (start 122.775 120.8258) (end 122.775 123) (width 0.25) (layer "F.Cu") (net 2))
 (segment (start 126.4267 112.35) (end 126.4267 112.306) (width 0.25) (layer "F.Cu") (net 2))
 (segment (start 126.4267 112.306) (end 121.419 107.2983) (width 0.25) (layer "F.Cu") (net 2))
 (segment (start 121.775 105) (end 121.775 106.9423) (width 0.25) (layer "F.Cu") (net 2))
 (segment (start 121.775 106.9423) (end 121.419 107.2983) (width 0.25) (layer "F.Cu") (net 2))
 (segment (start 107.95 104) (end 112.775 104) (width 0.25) (layer "F.Cu") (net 2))
 (segment (start 112.775 104) (end 113.775 105) (width 0.25) (layer "F.Cu") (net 2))
 (segment (start 118.25 108.0625) (end 118.25 107.2983) (width 0.25) (layer "F.Cu") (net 2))
 (segment (start 109.775 123.0231) (end 110.5536 123.8017) (width 0.25) (layer "F.Cu") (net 2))
 (segment (start 110.5536 123.8017) (end 111.9733 123.8017) (width 0.25) (layer "F.Cu") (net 2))
 (segment (start 111.9733 123.8017) (end 112.775 123) (width 0.25) (layer "F.Cu") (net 2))
 (segment (start 122.775 120.8258) (end 128.3342 120.8258) (width 0.25) (layer "F.Cu") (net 2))
 (segment (start 128.3342 120.8258) (end 133 116.16) (width 0.25) (layer "F.Cu") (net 2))
 (segment (start 116.25 108.0625) (end 116.25 107.5379) (width 0.25) (layer "F.Cu") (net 2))
 (segment (start 116.25 107.5379) (end 116.0104 107.2983) (width 0.25) (layer "F.Cu") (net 2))
 (segment (start 116.0104 107.2983) (end 115.4531 107.2983) (width 0.25) (layer "F.Cu") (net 2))
 (segment (start 115.4531 107.2983) (end 114.914 107.8374) (width 0.25) (layer "F.Cu") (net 2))
 (segment (start 114.914 107.8374) (end 114.2752 107.8374) (width 0.25) (layer "F.Cu") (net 2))
 (segment (start 114.2752 107.8374) (end 113.8132 108.2994) (width 0.25) (layer "F.Cu") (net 2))
 (segment (start 113.8132 108.2994) (end 113.8132 111.7643) (width 0.25) (layer "F.Cu") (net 2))
 (segment (start 113.8132 111.7643) (end 115.8415 113.7926) (width 0.25) (layer "F.Cu") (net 2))
 (segment (start 115.8415 113.7926) (end 115.9237 113.7926) (width 0.25) (layer "F.Cu") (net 2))
 (segment (start 115.9237 113.7926) (end 117.3233 115.1922) (width 0.25) (layer "F.Cu") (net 2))
 (segment (start 117.3233 115.1922) (end 117.3233 117.1134) (width 0.25) (layer "F.Cu") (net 2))
 (segment (start 117.3233 117.1134) (end 121.0357 120.8258) (width 0.25) (layer "F.Cu") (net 2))
 (segment (start 121.0357 120.8258) (end 122.775 120.8258) (width 0.25) (layer "F.Cu") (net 2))
 (segment (start 126.4267 112.35) (end 124.7767 114) (width 0.25) (layer "F.Cu") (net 2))
 (segment (start 133 116.16) (end 134.2176 114.9424) (width 0.25) (layer "F.Cu") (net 2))
 (segment (start 134.2176 114.9424) (end 134.2176 113.1367) (width 0.25) (layer "F.Cu") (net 2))
 (segment (start 134.2176 113.1367) (end 133.4309 112.35) (width 0.25) (layer "F.Cu") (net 2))
 (segment (start 133.4309 112.35) (end 126.4267 112.35) (width 0.25) (layer "F.Cu") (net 2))
 (segment (start 123.95 114) (end 124.7767 114) (width 0.25) (layer "F.Cu") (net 2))
 (segment (start 109.775 115) (end 109.775 123.0231) (width 0.25) (layer "F.Cu") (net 2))
 (segment (start 109.775 123.0231) (end 104.2581 128.54) (width 0.25) (layer "F.Cu") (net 2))
 (segment (start 104.2581 128.54) (end 104 128.54) (width 0.25) (layer "F.Cu") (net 2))
 (segment (start 119.7017 108.75) (end 122.05 111.0983) (width 0.25) (layer "F.Cu") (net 20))
 (segment (start 122.05 111.0983) (end 122.05 112.9483) (width 0.25) (layer "F.Cu") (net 20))
 (segment (start 118.9375 108.75) (end 119.7017 108.75) (width 0.25) (layer "F.Cu") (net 20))
 (segment (start 122.05 114) (end 122.05 112.9483) (width 0.25) (layer "F.Cu") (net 20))
 (segment (start 115.4 116.25) (end 115.4 117.2267) (width 0.25) (layer "F.Cu") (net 21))
 (segment (start 111.225 123) (end 111.225 121.4017) (width 0.25) (layer "F.Cu") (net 21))
 (segment (start 111.225 121.4017) (end 115.4 117.2267) (width 0.25) (layer "F.Cu") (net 21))
 (segment (start 115.4 115.2733) (end 112.9098 112.7831) (width 0.25) (layer "F.Cu") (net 21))
 (segment (start 112.9098 112.7831) (end 112.9098 107.9252) (width 0.25) (layer "F.Cu") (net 21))
 (segment (start 112.9098 107.9252) (end 114.4463 106.3887) (width 0.25) (layer "F.Cu") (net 21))
 (segment (start 114.4463 106.3887) (end 116.4917 106.3887) (width 0.25) (layer "F.Cu") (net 21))
 (segment (start 116.4917 106.3887) (end 117.25 107.147) (width 0.25) (layer "F.Cu") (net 21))
 (segment (start 117.25 107.147) (end 117.25 108.0625) (width 0.25) (layer "F.Cu") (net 21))
 (segment (start 115.4 116.25) (end 115.4 115.2733) (width 0.25) (layer "F.Cu") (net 21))
 (segment (start 115.4 121.75) (end 115.4 122.7267) (width 0.25) (layer "F.Cu") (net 22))
 (segment (start 121.225 123) (end 115.6733 123) (width 0.25) (layer "F.Cu") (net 22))
 (segment (start 115.6733 123) (end 115.4 122.7267) (width 0.25) (layer "F.Cu") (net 22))
 (segment (start 115.4 120.7733) (end 116.6767 119.4966) (width 0.25) (layer "F.Cu") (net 22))
 (segment (start 116.6767 119.4966) (end 116.6767 115.2666) (width 0.25) (layer "F.Cu") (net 22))
 (segment (start 116.6767 115.2666) (end 113.3615 111.9514) (width 0.25) (layer "F.Cu") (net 22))
 (segment (start 113.3615 111.9514) (end 113.3615 108.1123) (width 0.25) (layer "F.Cu") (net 22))
 (segment (start 113.3615 108.1123) (end 114.0881 107.3857) (width 0.25) (layer "F.Cu") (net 22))
 (segment (start 114.0881 107.3857) (end 114.7269 107.3857) (width 0.25) (layer "F.Cu") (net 22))
 (segment (start 114.7269 107.3857) (end 115.266 106.8466) (width 0.25) (layer "F.Cu") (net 22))
 (segment (start 115.266 106.8466) (end 116.2983 106.8466) (width 0.25) (layer "F.Cu") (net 22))
 (segment (start 116.2983 106.8466) (end 116.75 107.2983) (width 0.25) (layer "F.Cu") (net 22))
 (segment (start 115.4 121.75) (end 115.4 120.7733) (width 0.25) (layer "F.Cu") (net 22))
 (segment (start 116.75 108.0625) (end 116.75 107.2983) (width 0.25) (layer "F.Cu") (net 22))
 (segment (start 117.75 111.9375) (end 117.75 112.7017) (width 0.25) (layer "F.Cu") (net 13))
 (segment (start 133 113.62) (end 131.5683 115.0517) (width 0.25) (layer "F.Cu") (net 13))
 (segment (start 131.5683 115.0517) (end 120.1 115.0517) (width 0.25) (layer "F.Cu") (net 13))
 (segment (start 120.1 115.0517) (end 117.75 112.7017) (width 0.25) (layer "F.Cu") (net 13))
 (segment (start 109.825 111) (end 109.0983 111) (width 0.25) (layer "F.Cu") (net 14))
 (segment (start 108.225 115) (end 109.0983 114.1267) (width 0.25) (layer "F.Cu") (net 14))
 (segment (start 109.0983 114.1267) (end 109.0983 111) (width 0.25) (layer "F.Cu") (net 14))
 (segment (start 109.825 111) (end 110.5517 111) (width 0.25) (layer "F.Cu") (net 14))
 (segment (start 110.8142 111.2625) (end 110.5517 111) (width 0.25) (layer "F.Cu") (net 14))
 (segment (start 121.0595 111.6718) (end 111.2362 111.6718) (width 0.25) (layer "B.Cu") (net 14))
 (segment (start 111.2362 111.6718) (end 110.8269 111.2625) (width 0.25) (layer "B.Cu") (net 14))
 (segment (start 133 106) (end 131.8233 106) (width 0.25) (layer "B.Cu") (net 14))
 (segment (start 121.0595 111.6718) (end 120.7938 111.9375) (width 0.25) (layer "F.Cu") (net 14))
 (segment (start 120.7938 111.9375) (end 118.25 111.9375) (width 0.25) (layer "F.Cu") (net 14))
 (segment (start 131.8233 106) (end 126.1515 111.6718) (width 0.25) (layer "B.Cu") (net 14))
 (segment (start 126.1515 111.6718) (end 121.0595 111.6718) (width 0.25) (layer "B.Cu") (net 14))
 (via (at 116.1971 113.1724) (size 0.6) (drill 0.3) (layers "F.Cu" "B.Cu") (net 1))
 (via (at 110.8269 111.2625) (size 0.6) (drill 0.3) (layers "F.Cu" "B.Cu") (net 14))
 (via (at 121.0595 111.6718) (size 0.6) (drill 0.3) (layers "F.Cu" "B.Cu") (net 14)))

